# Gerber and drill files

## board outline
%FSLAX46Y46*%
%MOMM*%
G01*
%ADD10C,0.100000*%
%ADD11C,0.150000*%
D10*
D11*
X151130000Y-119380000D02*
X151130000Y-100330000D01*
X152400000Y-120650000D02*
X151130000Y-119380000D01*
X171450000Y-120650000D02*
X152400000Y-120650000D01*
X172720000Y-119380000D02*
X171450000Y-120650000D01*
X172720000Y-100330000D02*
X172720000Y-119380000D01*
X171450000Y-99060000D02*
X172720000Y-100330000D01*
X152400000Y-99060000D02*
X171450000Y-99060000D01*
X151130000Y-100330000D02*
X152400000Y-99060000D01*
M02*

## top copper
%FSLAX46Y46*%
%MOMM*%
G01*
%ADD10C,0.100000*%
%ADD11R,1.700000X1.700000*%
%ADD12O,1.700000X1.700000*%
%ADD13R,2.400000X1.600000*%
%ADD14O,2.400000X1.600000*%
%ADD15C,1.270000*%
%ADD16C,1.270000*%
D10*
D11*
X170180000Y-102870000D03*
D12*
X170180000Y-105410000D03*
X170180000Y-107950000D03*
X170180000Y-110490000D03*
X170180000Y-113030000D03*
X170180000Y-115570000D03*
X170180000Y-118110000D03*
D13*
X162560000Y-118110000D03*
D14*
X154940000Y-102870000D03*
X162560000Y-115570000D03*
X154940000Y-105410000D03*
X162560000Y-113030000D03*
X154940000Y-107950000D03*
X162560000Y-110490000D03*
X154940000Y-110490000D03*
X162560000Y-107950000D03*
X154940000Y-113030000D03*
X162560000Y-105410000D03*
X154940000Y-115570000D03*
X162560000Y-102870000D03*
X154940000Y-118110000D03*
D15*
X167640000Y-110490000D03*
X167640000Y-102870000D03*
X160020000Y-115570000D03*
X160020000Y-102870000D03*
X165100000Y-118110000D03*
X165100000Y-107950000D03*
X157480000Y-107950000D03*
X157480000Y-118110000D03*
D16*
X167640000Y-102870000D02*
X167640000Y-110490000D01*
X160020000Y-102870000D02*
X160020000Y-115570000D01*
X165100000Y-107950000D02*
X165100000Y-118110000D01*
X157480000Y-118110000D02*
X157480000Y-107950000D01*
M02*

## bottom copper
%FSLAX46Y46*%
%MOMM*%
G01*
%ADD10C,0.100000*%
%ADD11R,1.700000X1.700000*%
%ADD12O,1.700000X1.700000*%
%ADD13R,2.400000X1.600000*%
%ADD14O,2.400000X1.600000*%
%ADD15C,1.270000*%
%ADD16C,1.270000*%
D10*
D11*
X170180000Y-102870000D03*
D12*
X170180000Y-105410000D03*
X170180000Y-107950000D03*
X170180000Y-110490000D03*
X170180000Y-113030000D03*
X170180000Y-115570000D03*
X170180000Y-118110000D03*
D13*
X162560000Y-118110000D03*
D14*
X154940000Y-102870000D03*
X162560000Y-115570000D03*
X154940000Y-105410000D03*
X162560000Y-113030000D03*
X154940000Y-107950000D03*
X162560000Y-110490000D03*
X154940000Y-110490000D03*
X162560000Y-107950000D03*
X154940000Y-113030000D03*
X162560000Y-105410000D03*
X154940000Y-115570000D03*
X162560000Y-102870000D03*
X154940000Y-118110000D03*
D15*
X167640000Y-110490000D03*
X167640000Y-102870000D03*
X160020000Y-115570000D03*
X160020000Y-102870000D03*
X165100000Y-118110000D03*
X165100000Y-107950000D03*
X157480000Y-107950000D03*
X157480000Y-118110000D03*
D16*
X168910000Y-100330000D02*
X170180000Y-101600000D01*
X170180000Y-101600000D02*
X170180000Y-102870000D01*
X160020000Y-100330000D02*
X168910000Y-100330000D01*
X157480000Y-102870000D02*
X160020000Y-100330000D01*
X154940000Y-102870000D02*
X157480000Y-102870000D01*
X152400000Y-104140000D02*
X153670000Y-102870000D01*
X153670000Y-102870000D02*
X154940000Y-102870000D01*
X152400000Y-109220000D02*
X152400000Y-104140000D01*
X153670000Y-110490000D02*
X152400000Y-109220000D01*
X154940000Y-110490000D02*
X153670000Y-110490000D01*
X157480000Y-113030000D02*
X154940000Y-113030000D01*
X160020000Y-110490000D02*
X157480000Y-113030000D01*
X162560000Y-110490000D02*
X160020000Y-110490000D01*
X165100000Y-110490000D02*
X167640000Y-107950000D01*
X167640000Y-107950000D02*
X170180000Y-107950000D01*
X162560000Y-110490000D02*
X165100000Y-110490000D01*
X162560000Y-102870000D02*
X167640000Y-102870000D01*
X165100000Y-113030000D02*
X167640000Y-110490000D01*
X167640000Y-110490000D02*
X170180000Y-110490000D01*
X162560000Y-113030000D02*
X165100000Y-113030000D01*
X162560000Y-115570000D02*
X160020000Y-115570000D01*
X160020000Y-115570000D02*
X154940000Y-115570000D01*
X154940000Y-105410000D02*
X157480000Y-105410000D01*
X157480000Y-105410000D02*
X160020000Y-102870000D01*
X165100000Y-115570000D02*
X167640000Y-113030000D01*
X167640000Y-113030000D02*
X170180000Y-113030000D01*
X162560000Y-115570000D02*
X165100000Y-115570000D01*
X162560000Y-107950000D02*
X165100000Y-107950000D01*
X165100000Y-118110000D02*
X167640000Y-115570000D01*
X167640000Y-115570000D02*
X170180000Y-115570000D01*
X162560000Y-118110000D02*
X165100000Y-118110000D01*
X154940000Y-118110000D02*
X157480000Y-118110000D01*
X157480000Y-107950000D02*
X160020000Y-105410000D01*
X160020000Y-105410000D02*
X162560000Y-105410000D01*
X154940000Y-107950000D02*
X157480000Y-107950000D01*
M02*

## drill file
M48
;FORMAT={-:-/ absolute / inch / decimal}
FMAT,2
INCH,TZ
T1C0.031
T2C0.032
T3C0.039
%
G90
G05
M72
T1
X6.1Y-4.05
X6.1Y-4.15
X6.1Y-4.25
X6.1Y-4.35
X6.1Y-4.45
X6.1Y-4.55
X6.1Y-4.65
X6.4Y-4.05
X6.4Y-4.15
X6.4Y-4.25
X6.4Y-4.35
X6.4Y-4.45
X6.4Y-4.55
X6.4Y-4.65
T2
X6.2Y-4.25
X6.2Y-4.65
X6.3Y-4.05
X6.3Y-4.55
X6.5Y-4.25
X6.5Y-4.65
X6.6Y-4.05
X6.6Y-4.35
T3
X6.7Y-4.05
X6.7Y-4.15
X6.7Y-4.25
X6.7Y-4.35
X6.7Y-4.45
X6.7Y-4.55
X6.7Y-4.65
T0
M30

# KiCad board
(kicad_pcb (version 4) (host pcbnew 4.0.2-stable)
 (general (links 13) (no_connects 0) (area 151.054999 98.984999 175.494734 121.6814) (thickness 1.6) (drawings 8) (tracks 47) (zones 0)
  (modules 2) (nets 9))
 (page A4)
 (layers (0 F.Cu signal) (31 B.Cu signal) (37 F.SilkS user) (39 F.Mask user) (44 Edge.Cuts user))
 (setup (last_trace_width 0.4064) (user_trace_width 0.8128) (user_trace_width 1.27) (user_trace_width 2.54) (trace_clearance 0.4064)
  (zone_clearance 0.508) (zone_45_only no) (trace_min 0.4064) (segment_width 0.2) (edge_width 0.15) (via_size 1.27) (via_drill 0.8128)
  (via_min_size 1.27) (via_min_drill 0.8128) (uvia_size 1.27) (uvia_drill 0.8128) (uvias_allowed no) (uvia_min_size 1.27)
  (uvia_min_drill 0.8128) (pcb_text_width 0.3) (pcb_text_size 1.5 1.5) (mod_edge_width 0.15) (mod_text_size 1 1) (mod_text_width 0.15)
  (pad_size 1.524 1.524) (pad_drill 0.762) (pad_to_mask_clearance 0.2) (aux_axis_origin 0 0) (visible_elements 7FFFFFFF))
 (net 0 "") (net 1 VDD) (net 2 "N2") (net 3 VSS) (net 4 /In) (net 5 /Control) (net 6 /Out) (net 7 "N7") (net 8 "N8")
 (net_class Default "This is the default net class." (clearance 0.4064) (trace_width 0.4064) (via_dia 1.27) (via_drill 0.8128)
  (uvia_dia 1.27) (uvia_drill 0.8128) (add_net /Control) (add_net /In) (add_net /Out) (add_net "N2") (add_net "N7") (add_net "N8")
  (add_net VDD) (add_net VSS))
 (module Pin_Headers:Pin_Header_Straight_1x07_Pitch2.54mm (layer F.Cu) (at 170.18 102.87)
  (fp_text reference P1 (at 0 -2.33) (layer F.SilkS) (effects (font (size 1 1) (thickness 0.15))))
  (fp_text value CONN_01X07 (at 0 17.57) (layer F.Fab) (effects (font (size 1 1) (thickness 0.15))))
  (pad 1 thru_hole rect (at 0 0) (size 1.7 1.7) (drill 1) (layers *.Cu *.Mask) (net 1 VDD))
  (pad 2 thru_hole oval (at 0 2.54) (size 1.7 1.7) (drill 1) (layers *.Cu *.Mask) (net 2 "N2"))
  (pad 3 thru_hole oval (at 0 5.08) (size 1.7 1.7) (drill 1) (layers *.Cu *.Mask) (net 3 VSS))
  (pad 4 thru_hole oval (at 0 7.62) (size 1.7 1.7) (drill 1) (layers *.Cu *.Mask) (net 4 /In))
  (pad 5 thru_hole oval (at 0 10.16) (size 1.7 1.7) (drill 1) (layers *.Cu *.Mask) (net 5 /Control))
  (pad 6 thru_hole oval (at 0 12.7) (size 1.7 1.7) (drill 1) (layers *.Cu *.Mask) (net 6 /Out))
  (pad 7 thru_hole oval (at 0 15.24) (size 1.7 1.7) (drill 1) (layers *.Cu *.Mask) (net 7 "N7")))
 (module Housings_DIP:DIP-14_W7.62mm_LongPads (layer F.Cu) (at 162.56 118.11 180)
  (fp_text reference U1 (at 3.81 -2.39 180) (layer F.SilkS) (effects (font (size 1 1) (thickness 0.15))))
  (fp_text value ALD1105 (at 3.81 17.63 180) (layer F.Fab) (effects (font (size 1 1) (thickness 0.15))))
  (pad 1 thru_hole rect (at 0 0 180) (size 2.4 1.6) (drill 0.8) (layers *.Cu *.Mask) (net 6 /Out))
  (pad 8 thru_hole oval (at 7.62 15.24 180) (size 2.4 1.6) (drill 0.8) (layers *.Cu *.Mask) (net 1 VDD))
  (pad 2 thru_hole oval (at 0 2.54 180) (size 2.4 1.6) (drill 0.8) (layers *.Cu *.Mask) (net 5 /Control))
  (pad 9 thru_hole oval (at 7.62 12.7 180) (size 2.4 1.6) (drill 0.8) (layers *.Cu *.Mask) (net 5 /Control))
  (pad 3 thru_hole oval (at 0 5.08 180) (size 2.4 1.6) (drill 0.8) (layers *.Cu *.Mask) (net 4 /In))
  (pad 10 thru_hole oval (at 7.62 10.16 180) (size 2.4 1.6) (drill 0.8) (layers *.Cu *.Mask) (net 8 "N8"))
  (pad 4 thru_hole oval (at 0 7.62 180) (size 2.4 1.6) (drill 0.8) (layers *.Cu *.Mask) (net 3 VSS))
  (pad 11 thru_hole oval (at 7.62 7.62 180) (size 2.4 1.6) (drill 0.8) (layers *.Cu *.Mask) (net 1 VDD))
  (pad 5 thru_hole oval (at 0 10.16 180) (size 2.4 1.6) (drill 0.8) (layers *.Cu *.Mask) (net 6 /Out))
  (pad 12 thru_hole oval (at 7.62 5.08 180) (size 2.4 1.6) (drill 0.8) (layers *.Cu *.Mask) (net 3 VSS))
  (pad 6 thru_hole oval (at 0 12.7 180) (size 2.4 1.6) (drill 0.8) (layers *.Cu *.Mask) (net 8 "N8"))
  (pad 13 thru_hole oval (at 7.62 2.54 180) (size 2.4 1.6) (drill 0.8) (layers *.Cu *.Mask) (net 5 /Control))
  (pad 7 thru_hole oval (at 0 15.24 180) (size 2.4 1.6) (drill 0.8) (layers *.Cu *.Mask) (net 4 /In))
  (pad 14 thru_hole oval (at 7.62 0 180) (size 2.4 1.6) (drill 0.8) (layers *.Cu *.Mask) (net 8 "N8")))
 (gr_line (start 151.13 119.38) (end 151.13 100.33) (layer Edge.Cuts) (width 0.15))
 (gr_line (start 152.4 120.65) (end 151.13 119.38) (layer Edge.Cuts) (width 0.15))
 (gr_line (start 171.45 120.65) (end 152.4 120.65) (layer Edge.Cuts) (width 0.15))
 (gr_line (start 172.72 119.38) (end 171.45 120.65) (layer Edge.Cuts) (width 0.15))
 (gr_line (start 172.72 100.33) (end 172.72 119.38) (layer Edge.Cuts) (width 0.15))
 (gr_line (start 171.45 99.06) (end 172.72 100.33) (layer Edge.Cuts) (width 0.15))
 (gr_line (start 152.4 99.06) (end 171.45 99.06) (layer Edge.Cuts) (width 0.15))
 (gr_line (start 151.13 100.33) (end 152.4 99.06) (layer Edge.Cuts) (width 0.15))
 (segment (start 168.91 100.33) (end 170.18 101.6) (width 1.27) (layer B.Cu) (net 1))
 (segment (start 170.18 101.6) (end 170.18 102.87) (width 1.27) (layer B.Cu) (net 1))
 (segment (start 160.02 100.33) (end 168.91 100.33) (width 1.27) (layer B.Cu) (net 1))
 (segment (start 157.48 102.87) (end 160.02 100.33) (width 1.27) (layer B.Cu) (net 1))
 (segment (start 154.94 102.87) (end 157.48 102.87) (width 1.27) (layer B.Cu) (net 1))
 (segment (start 152.4 104.14) (end 153.67 102.87) (width 1.27) (layer B.Cu) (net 1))
 (segment (start 153.67 102.87) (end 154.94 102.87) (width 1.27) (layer B.Cu) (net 1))
 (segment (start 152.4 109.22) (end 152.4 104.14) (width 1.27) (layer B.Cu) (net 1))
 (segment (start 153.67 110.49) (end 152.4 109.22) (width 1.27) (layer B.Cu) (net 1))
 (segment (start 154.94 110.49) (end 153.67 110.49) (width 1.27) (layer B.Cu) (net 1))
 (segment (start 157.48 113.03) (end 154.94 113.03) (width 1.27) (layer B.Cu) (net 3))
 (segment (start 160.02 110.49) (end 157.48 113.03) (width 1.27) (layer B.Cu) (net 3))
 (segment (start 162.56 110.49) (end 160.02 110.49) (width 1.27) (layer B.Cu) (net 3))
 (segment (start 165.1 110.49) (end 167.64 107.95) (width 1.27) (layer B.Cu) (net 3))
 (segment (start 167.64 107.95) (end 170.18 107.95) (width 1.27) (layer B.Cu) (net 3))
 (segment (start 162.56 110.49) (end 165.1 110.49) (width 1.27) (layer B.Cu) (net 3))
 (segment (start 167.64 102.87) (end 167.64 110.49) (width 1.27) (layer F.Cu) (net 4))
 (via (at 167.64 110.49) (size 1.27) (drill 0.8128) (layers F.Cu B.Cu) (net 4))
 (segment (start 162.56 102.87) (end 167.64 102.87) (width 1.27) (layer B.Cu) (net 4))
 (via (at 167.64 102.87) (size 1.27) (drill 0.8128) (layers F.Cu B.Cu) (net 4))
 (segment (start 165.1 113.03) (end 167.64 110.49) (width 1.27) (layer B.Cu) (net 4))
 (segment (start 167.64 110.49) (end 170.18 110.49) (width 1.27) (layer B.Cu) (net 4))
 (segment (start 162.56 113.03) (end 165.1 113.03) (width 1.27) (layer B.Cu) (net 4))
 (segment (start 162.56 115.57) (end 160.02 115.57) (width 1.27) (layer B.Cu) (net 5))
 (segment (start 160.02 115.57) (end 154.94 115.57) (width 1.27) (layer B.Cu) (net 5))
 (segment (start 160.02 102.87) (end 160.02 115.57) (width 1.27) (layer F.Cu) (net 5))
 (via (at 160.02 115.57) (size 1.27) (drill 0.8128) (layers F.Cu B.Cu) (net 5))
 (segment (start 154.94 105.41) (end 157.48 105.41) (width 1.27) (layer B.Cu) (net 5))
 (segment (start 157.48 105.41) (end 160.02 102.87) (width 1.27) (layer B.Cu) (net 5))
 (via (at 160.02 102.87) (size 1.27) (drill 0.8128) (layers F.Cu B.Cu) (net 5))
 (segment (start 165.1 115.57) (end 167.64 113.03) (width 1.27) (layer B.Cu) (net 5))
 (segment (start 167.64 113.03) (end 170.18 113.03) (width 1.27) (layer B.Cu) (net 5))
 (segment (start 162.56 115.57) (end 165.1 115.57) (width 1.27) (layer B.Cu) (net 5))
 (segment (start 165.1 107.95) (end 165.1 118.11) (width 1.27) (layer F.Cu) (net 6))
 (via (at 165.1 118.11) (size 1.27) (drill 0.8128) (layers F.Cu B.Cu) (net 6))
 (segment (start 162.56 107.95) (end 165.1 107.95) (width 1.27) (layer B.Cu) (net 6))
 (via (at 165.1 107.95) (size 1.27) (drill 0.8128) (layers F.Cu B.Cu) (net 6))
 (segment (start 165.1 118.11) (end 167.64 115.57) (width 1.27) (layer B.Cu) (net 6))
 (segment (start 167.64 115.57) (end 170.18 115.57) (width 1.27) (layer B.Cu) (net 6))
 (segment (start 162.56 118.11) (end 165.1 118.11) (width 1.27) (layer B.Cu) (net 6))
 (segment (start 157.48 118.11) (end 157.48 107.95) (width 1.27) (layer F.Cu) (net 8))
 (via (at 157.48 107.95) (size 1.27) (drill 0.8128) (layers F.Cu B.Cu) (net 8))
 (segment (start 154.94 118.11) (end 157.48 118.11) (width 1.27) (layer B.Cu) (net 8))
 (via (at 157.48 118.11) (size 1.27) (drill 0.8128) (layers F.Cu B.Cu) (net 8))
 (segment (start 157.48 107.95) (end 160.02 105.41) (width 1.27) (layer B.Cu) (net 8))
 (segment (start 160.02 105.41) (end 162.56 105.41) (width 1.27) (layer B.Cu) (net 8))
 (segment (start 154.94 107.95) (end 157.48 107.95) (width 1.27) (layer B.Cu) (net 8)))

